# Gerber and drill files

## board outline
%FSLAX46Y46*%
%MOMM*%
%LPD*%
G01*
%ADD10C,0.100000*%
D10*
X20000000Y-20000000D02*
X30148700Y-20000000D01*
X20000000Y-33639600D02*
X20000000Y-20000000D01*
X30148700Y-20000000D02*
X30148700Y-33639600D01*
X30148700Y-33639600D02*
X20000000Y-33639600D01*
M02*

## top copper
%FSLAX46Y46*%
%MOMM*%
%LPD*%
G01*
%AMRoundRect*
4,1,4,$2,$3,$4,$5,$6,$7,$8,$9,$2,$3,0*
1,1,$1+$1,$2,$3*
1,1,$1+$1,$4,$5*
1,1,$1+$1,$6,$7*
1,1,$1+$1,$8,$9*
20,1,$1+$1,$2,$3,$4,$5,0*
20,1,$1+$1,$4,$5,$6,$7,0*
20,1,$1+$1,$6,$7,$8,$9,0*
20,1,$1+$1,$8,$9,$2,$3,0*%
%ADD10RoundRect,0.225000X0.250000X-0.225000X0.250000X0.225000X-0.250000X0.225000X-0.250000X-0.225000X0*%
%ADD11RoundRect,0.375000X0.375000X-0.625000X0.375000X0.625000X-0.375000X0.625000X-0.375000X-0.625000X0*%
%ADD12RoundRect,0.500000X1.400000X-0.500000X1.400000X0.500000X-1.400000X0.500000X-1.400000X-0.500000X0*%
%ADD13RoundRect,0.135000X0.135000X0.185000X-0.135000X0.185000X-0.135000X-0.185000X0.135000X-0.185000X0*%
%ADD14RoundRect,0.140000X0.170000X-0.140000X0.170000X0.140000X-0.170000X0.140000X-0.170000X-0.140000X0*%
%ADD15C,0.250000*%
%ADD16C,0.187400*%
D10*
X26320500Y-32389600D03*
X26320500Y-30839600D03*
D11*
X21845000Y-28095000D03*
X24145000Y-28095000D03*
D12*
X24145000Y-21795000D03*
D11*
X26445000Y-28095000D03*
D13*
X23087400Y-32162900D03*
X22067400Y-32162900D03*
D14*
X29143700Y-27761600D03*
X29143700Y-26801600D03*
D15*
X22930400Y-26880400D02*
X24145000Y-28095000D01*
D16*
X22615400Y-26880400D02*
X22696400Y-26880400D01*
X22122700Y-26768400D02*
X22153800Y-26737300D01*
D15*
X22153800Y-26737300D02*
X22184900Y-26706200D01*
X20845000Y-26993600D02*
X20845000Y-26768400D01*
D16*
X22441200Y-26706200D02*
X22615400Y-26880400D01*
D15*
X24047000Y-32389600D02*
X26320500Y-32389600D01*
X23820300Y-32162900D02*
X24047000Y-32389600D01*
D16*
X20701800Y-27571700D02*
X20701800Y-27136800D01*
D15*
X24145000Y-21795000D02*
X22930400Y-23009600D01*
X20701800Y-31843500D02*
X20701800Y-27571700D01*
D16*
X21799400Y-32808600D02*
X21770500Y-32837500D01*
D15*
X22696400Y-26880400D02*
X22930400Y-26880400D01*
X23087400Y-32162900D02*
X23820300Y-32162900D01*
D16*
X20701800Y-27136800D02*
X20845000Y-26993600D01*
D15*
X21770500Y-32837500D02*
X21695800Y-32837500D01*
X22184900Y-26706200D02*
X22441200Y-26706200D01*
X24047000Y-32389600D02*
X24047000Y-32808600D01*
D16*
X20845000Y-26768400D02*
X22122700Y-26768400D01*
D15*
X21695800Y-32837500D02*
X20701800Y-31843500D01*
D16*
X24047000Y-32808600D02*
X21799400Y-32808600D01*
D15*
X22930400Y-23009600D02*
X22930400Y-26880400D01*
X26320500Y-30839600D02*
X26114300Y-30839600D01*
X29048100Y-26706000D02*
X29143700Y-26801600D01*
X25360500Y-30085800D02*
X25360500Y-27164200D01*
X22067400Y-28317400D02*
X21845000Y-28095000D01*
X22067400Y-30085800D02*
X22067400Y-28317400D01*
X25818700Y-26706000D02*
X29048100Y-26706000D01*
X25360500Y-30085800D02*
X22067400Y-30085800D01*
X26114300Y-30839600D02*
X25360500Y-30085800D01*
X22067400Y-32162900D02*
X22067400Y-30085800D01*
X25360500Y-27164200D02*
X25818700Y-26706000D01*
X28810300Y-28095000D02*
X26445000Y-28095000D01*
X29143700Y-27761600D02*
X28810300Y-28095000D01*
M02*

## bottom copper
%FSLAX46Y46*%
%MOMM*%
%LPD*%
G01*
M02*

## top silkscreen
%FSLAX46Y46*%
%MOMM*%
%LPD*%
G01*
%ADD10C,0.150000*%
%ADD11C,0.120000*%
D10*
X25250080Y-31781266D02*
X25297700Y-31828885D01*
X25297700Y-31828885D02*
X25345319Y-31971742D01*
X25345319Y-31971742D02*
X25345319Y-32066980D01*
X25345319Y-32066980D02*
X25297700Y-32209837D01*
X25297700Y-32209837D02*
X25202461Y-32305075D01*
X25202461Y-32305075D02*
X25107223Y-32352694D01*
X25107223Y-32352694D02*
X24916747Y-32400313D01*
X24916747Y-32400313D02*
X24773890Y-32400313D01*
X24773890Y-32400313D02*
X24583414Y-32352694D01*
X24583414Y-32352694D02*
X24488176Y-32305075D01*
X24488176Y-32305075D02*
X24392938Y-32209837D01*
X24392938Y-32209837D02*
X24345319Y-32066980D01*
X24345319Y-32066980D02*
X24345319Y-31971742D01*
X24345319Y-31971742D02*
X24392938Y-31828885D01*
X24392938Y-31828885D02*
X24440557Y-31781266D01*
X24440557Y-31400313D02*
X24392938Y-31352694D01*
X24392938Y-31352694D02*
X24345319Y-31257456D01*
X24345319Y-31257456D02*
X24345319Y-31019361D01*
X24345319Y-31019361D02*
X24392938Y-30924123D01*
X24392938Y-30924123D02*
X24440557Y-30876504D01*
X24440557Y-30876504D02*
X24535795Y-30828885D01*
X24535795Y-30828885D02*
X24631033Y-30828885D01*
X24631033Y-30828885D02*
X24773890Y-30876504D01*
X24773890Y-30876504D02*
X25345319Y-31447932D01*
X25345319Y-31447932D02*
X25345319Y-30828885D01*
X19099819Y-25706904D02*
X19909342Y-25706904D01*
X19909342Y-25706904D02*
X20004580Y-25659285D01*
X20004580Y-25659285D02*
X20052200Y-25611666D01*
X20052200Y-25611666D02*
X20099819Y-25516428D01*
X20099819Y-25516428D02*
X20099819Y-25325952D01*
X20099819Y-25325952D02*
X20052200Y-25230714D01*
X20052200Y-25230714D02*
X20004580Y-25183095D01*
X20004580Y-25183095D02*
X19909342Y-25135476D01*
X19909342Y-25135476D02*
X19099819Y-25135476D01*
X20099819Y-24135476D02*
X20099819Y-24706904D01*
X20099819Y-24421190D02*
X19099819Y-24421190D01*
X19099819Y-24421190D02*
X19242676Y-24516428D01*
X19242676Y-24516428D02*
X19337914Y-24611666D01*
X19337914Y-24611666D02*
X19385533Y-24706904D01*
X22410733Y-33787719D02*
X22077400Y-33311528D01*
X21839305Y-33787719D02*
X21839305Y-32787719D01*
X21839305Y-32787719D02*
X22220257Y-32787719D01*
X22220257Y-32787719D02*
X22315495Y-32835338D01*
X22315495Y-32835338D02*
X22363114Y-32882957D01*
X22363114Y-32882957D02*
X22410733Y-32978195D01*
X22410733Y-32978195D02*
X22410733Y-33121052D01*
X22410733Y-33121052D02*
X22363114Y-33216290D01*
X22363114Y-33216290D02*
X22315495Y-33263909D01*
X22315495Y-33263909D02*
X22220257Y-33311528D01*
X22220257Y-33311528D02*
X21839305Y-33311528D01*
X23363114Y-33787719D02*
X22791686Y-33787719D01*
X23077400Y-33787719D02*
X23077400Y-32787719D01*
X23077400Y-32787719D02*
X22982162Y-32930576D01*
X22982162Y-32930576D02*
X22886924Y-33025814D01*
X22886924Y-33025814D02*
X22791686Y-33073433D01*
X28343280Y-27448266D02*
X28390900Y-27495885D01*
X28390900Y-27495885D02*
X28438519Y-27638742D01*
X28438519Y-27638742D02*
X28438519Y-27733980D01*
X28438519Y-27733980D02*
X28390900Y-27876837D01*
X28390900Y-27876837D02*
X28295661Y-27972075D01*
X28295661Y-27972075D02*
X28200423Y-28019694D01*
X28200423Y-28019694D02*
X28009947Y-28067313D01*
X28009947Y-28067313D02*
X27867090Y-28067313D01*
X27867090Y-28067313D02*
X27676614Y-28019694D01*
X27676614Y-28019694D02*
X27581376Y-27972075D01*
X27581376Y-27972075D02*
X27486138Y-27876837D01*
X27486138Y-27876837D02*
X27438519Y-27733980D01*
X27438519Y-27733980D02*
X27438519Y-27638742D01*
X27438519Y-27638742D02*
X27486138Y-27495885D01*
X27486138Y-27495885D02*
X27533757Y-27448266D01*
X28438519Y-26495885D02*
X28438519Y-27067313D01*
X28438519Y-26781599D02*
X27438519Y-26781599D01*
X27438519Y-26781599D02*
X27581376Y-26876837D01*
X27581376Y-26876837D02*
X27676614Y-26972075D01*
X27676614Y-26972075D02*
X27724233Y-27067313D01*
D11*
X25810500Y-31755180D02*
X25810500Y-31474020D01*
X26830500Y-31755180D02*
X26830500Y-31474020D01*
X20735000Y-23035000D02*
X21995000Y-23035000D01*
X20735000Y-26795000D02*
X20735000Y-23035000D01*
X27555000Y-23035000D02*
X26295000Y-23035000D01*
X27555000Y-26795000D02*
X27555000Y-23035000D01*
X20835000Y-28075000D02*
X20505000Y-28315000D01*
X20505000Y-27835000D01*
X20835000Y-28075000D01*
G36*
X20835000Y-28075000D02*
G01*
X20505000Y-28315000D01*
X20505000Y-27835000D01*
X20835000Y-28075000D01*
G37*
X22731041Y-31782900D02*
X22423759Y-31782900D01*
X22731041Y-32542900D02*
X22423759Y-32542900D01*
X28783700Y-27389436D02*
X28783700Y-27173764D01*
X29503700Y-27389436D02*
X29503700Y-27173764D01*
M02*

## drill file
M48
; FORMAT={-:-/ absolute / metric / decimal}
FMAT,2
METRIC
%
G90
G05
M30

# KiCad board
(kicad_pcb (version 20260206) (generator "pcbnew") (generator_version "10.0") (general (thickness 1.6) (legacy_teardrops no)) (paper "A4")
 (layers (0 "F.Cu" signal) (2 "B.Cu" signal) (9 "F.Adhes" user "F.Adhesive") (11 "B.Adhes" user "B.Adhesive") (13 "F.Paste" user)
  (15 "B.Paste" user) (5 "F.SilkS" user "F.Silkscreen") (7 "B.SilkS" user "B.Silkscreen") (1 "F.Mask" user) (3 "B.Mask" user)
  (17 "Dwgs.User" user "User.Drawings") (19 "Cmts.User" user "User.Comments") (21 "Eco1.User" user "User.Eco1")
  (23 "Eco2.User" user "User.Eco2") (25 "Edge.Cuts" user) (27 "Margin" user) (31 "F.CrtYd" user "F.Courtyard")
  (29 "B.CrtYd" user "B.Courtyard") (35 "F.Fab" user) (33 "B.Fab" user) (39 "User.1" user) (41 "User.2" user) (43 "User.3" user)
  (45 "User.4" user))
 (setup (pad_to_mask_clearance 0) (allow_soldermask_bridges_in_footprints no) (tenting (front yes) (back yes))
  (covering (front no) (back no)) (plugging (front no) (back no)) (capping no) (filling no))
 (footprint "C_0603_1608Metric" (layer "F.Cu") (at 26.3205 31.6146 90)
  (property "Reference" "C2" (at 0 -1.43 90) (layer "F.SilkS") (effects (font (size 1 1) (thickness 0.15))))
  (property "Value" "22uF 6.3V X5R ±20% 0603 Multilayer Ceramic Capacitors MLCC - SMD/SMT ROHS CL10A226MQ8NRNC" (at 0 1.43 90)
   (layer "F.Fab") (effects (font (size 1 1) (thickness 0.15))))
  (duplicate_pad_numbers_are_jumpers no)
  (fp_line (start -0.14058 -0.51) (end 0.14058 -0.51) (stroke (width 0.12) (type solid)) (layer "F.SilkS"))
  (fp_line (start -0.14058 0.51) (end 0.14058 0.51) (stroke (width 0.12) (type solid)) (layer "F.SilkS"))
  (pad "1" smd roundrect (at -0.775 0 90) (size 0.9 0.95) (layers "F.Cu" "F.Mask" "F.Paste") (roundrect_rratio 0.25) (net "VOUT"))
  (pad "2" smd roundrect (at 0.775 0 90) (size 0.9 0.95) (layers "F.Cu" "F.Mask" "F.Paste") (roundrect_rratio 0.25) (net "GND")))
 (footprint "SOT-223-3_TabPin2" (layer "F.Cu") (at 24.145 24.945 90)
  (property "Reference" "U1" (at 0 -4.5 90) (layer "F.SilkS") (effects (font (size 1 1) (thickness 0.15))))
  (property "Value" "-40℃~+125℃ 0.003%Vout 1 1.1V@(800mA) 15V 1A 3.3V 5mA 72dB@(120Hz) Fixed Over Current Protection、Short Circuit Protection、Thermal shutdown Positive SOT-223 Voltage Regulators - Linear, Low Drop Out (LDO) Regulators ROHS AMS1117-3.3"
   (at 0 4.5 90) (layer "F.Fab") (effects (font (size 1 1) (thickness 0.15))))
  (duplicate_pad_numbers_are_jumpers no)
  (fp_line (start 1.91 -3.41) (end 1.91 -2.15) (stroke (width 0.12) (type solid)) (layer "F.SilkS"))
  (fp_line (start -1.85 -3.41) (end 1.91 -3.41) (stroke (width 0.12) (type solid)) (layer "F.SilkS"))
  (fp_line (start 1.91 3.41) (end 1.91 2.15) (stroke (width 0.12) (type solid)) (layer "F.SilkS"))
  (fp_line (start -1.85 3.41) (end 1.91 3.41) (stroke (width 0.12) (type solid)) (layer "F.SilkS"))
  (fp_poly
   (pts (xy -3.13 -3.31) (xy -3.37 -3.64) (xy -2.89 -3.64) (xy -3.13 -3.31)) (stroke (width 0.12) (type solid)) (fill yes) (layer "F.SilkS"))
  (pad "1" smd roundrect (at -3.15 -2.3 90) (size 2 1.5) (layers "F.Cu" "F.Mask" "F.Paste") (roundrect_rratio 0.25) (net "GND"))
  (pad "2" smd roundrect (at -3.15 0 90) (size 2 1.5) (layers "F.Cu" "F.Mask" "F.Paste") (roundrect_rratio 0.25) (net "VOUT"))
  (pad "2" smd roundrect (at 3.15 0 90) (size 2 3.8) (layers "F.Cu" "F.Mask" "F.Paste") (roundrect_rratio 0.25) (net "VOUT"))
  (pad "3" smd roundrect (at -3.15 2.3 90) (size 2 1.5) (layers "F.Cu" "F.Mask" "F.Paste") (roundrect_rratio 0.25) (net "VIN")))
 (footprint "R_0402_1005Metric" (layer "F.Cu") (at 22.5774 32.1629 180)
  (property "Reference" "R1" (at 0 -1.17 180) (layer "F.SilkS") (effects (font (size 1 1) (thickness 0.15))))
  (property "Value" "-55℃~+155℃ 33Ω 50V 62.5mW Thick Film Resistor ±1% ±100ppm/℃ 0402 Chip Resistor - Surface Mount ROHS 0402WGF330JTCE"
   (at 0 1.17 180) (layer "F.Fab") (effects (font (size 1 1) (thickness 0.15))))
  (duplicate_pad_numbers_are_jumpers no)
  (fp_line (start -0.153641 0.38) (end 0.153641 0.38) (stroke (width 0.12) (type solid)) (layer "F.SilkS"))
  (fp_line (start -0.153641 -0.38) (end 0.153641 -0.38) (stroke (width 0.12) (type solid)) (layer "F.SilkS"))
  (pad "1" smd roundrect (at -0.51 0 180) (size 0.54 0.64) (layers "F.Cu" "F.Mask" "F.Paste") (roundrect_rratio 0.25) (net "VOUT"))
  (pad "2" smd roundrect (at 0.51 0 180) (size 0.54 0.64) (layers "F.Cu" "F.Mask" "F.Paste") (roundrect_rratio 0.25) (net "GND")))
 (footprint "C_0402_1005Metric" (layer "F.Cu") (at 29.1437 27.2816 90)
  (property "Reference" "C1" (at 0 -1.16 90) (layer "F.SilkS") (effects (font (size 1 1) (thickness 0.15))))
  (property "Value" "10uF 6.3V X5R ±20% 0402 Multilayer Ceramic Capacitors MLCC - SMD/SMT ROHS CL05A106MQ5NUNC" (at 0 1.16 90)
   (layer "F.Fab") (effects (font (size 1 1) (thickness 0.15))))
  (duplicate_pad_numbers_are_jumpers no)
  (fp_line (start -0.107836 -0.36) (end 0.107836 -0.36) (stroke (width 0.12) (type solid)) (layer "F.SilkS"))
  (fp_line (start -0.107836 0.36) (end 0.107836 0.36) (stroke (width 0.12) (type solid)) (layer "F.SilkS"))
  (pad "1" smd roundrect (at -0.48 0 90) (size 0.56 0.62) (layers "F.Cu" "F.Mask" "F.Paste") (roundrect_rratio 0.25) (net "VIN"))
  (pad "2" smd roundrect (at 0.48 0 90) (size 0.56 0.62) (layers "F.Cu" "F.Mask" "F.Paste") (roundrect_rratio 0.25) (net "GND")))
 (gr_line (start 20 20) (end 30.1487 20) (stroke (width 0.1) (type default)) (layer "Edge.Cuts"))
 (gr_line (start 20 33.6396) (end 20 20) (stroke (width 0.1) (type default)) (layer "Edge.Cuts"))
 (gr_line (start 30.1487 20) (end 30.1487 33.6396) (stroke (width 0.1) (type default)) (layer "Edge.Cuts"))
 (gr_line (start 30.1487 33.6396) (end 20 33.6396) (stroke (width 0.1) (type default)) (layer "Edge.Cuts"))
 (segment (start 22.9304 26.8804) (end 24.145 28.095) (width 0.25) (layer "F.Cu") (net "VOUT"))
 (segment (start 22.6154 26.8804) (end 22.6964 26.8804) (width 0.1874) (layer "F.Cu") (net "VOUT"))
 (segment (start 22.1227 26.7684) (end 22.1538 26.7373) (width 0.1874) (layer "F.Cu") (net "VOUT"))
 (segment (start 22.1538 26.7373) (end 22.1849 26.7062) (width 0.25) (layer "F.Cu") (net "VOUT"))
 (segment (start 20.845 26.9936) (end 20.845 26.7684) (width 0.25) (layer "F.Cu") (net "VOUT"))
 (segment (start 22.4412 26.7062) (end 22.6154 26.8804) (width 0.1874) (layer "F.Cu") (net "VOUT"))
 (segment (start 24.047 32.3896) (end 26.3205 32.3896) (width 0.25) (layer "F.Cu") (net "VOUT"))
 (segment (start 23.8203 32.1629) (end 24.047 32.3896) (width 0.25) (layer "F.Cu") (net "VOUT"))
 (segment (start 20.7018 27.5717) (end 20.7018 27.1368) (width 0.1874) (layer "F.Cu") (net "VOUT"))
 (segment (start 24.145 21.795) (end 22.9304 23.0096) (width 0.25) (layer "F.Cu") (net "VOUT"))
 (segment (start 20.7018 31.8435) (end 20.7018 27.5717) (width 0.25) (layer "F.Cu") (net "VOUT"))
 (segment (start 21.7994 32.8086) (end 21.7705 32.8375) (width 0.1874) (layer "F.Cu") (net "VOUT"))
 (segment (start 22.6964 26.8804) (end 22.9304 26.8804) (width 0.25) (layer "F.Cu") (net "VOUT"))
 (segment (start 23.0874 32.1629) (end 23.8203 32.1629) (width 0.25) (layer "F.Cu") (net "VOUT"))
 (segment (start 20.7018 27.1368) (end 20.845 26.9936) (width 0.1874) (layer "F.Cu") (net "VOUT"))
 (segment (start 21.7705 32.8375) (end 21.6958 32.8375) (width 0.25) (layer "F.Cu") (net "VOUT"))
 (segment (start 22.1849 26.7062) (end 22.4412 26.7062) (width 0.25) (layer "F.Cu") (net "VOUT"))
 (segment (start 24.047 32.3896) (end 24.047 32.8086) (width 0.25) (layer "F.Cu") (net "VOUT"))
 (segment (start 20.845 26.7684) (end 22.1227 26.7684) (width 0.1874) (layer "F.Cu") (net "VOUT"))
 (segment (start 21.6958 32.8375) (end 20.7018 31.8435) (width 0.25) (layer "F.Cu") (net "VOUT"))
 (segment (start 24.047 32.8086) (end 21.7994 32.8086) (width 0.1874) (layer "F.Cu") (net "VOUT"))
 (segment (start 22.9304 23.0096) (end 22.9304 26.8804) (width 0.25) (layer "F.Cu") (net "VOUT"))
 (segment (start 26.3205 30.8396) (end 26.1143 30.8396) (width 0.25) (layer "F.Cu") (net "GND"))
 (segment (start 29.0481 26.706) (end 29.1437 26.8016) (width 0.25) (layer "F.Cu") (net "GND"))
 (segment (start 25.3605 30.0858) (end 25.3605 27.1642) (width 0.25) (layer "F.Cu") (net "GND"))
 (segment (start 22.0674 28.3174) (end 21.845 28.095) (width 0.25) (layer "F.Cu") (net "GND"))
 (segment (start 22.0674 30.0858) (end 22.0674 28.3174) (width 0.25) (layer "F.Cu") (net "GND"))
 (segment (start 25.8187 26.706) (end 29.0481 26.706) (width 0.25) (layer "F.Cu") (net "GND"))
 (segment (start 25.3605 30.0858) (end 22.0674 30.0858) (width 0.25) (layer "F.Cu") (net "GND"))
 (segment (start 26.1143 30.8396) (end 25.3605 30.0858) (width 0.25) (layer "F.Cu") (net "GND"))
 (segment (start 22.0674 32.1629) (end 22.0674 30.0858) (width 0.25) (layer "F.Cu") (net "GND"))
 (segment (start 25.3605 27.1642) (end 25.8187 26.706) (width 0.25) (layer "F.Cu") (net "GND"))
 (segment (start 28.8103 28.095) (end 26.445 28.095) (width 0.25) (layer "F.Cu") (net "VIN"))
 (segment (start 29.1437 27.7616) (end 28.8103 28.095) (width 0.25) (layer "F.Cu") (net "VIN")))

